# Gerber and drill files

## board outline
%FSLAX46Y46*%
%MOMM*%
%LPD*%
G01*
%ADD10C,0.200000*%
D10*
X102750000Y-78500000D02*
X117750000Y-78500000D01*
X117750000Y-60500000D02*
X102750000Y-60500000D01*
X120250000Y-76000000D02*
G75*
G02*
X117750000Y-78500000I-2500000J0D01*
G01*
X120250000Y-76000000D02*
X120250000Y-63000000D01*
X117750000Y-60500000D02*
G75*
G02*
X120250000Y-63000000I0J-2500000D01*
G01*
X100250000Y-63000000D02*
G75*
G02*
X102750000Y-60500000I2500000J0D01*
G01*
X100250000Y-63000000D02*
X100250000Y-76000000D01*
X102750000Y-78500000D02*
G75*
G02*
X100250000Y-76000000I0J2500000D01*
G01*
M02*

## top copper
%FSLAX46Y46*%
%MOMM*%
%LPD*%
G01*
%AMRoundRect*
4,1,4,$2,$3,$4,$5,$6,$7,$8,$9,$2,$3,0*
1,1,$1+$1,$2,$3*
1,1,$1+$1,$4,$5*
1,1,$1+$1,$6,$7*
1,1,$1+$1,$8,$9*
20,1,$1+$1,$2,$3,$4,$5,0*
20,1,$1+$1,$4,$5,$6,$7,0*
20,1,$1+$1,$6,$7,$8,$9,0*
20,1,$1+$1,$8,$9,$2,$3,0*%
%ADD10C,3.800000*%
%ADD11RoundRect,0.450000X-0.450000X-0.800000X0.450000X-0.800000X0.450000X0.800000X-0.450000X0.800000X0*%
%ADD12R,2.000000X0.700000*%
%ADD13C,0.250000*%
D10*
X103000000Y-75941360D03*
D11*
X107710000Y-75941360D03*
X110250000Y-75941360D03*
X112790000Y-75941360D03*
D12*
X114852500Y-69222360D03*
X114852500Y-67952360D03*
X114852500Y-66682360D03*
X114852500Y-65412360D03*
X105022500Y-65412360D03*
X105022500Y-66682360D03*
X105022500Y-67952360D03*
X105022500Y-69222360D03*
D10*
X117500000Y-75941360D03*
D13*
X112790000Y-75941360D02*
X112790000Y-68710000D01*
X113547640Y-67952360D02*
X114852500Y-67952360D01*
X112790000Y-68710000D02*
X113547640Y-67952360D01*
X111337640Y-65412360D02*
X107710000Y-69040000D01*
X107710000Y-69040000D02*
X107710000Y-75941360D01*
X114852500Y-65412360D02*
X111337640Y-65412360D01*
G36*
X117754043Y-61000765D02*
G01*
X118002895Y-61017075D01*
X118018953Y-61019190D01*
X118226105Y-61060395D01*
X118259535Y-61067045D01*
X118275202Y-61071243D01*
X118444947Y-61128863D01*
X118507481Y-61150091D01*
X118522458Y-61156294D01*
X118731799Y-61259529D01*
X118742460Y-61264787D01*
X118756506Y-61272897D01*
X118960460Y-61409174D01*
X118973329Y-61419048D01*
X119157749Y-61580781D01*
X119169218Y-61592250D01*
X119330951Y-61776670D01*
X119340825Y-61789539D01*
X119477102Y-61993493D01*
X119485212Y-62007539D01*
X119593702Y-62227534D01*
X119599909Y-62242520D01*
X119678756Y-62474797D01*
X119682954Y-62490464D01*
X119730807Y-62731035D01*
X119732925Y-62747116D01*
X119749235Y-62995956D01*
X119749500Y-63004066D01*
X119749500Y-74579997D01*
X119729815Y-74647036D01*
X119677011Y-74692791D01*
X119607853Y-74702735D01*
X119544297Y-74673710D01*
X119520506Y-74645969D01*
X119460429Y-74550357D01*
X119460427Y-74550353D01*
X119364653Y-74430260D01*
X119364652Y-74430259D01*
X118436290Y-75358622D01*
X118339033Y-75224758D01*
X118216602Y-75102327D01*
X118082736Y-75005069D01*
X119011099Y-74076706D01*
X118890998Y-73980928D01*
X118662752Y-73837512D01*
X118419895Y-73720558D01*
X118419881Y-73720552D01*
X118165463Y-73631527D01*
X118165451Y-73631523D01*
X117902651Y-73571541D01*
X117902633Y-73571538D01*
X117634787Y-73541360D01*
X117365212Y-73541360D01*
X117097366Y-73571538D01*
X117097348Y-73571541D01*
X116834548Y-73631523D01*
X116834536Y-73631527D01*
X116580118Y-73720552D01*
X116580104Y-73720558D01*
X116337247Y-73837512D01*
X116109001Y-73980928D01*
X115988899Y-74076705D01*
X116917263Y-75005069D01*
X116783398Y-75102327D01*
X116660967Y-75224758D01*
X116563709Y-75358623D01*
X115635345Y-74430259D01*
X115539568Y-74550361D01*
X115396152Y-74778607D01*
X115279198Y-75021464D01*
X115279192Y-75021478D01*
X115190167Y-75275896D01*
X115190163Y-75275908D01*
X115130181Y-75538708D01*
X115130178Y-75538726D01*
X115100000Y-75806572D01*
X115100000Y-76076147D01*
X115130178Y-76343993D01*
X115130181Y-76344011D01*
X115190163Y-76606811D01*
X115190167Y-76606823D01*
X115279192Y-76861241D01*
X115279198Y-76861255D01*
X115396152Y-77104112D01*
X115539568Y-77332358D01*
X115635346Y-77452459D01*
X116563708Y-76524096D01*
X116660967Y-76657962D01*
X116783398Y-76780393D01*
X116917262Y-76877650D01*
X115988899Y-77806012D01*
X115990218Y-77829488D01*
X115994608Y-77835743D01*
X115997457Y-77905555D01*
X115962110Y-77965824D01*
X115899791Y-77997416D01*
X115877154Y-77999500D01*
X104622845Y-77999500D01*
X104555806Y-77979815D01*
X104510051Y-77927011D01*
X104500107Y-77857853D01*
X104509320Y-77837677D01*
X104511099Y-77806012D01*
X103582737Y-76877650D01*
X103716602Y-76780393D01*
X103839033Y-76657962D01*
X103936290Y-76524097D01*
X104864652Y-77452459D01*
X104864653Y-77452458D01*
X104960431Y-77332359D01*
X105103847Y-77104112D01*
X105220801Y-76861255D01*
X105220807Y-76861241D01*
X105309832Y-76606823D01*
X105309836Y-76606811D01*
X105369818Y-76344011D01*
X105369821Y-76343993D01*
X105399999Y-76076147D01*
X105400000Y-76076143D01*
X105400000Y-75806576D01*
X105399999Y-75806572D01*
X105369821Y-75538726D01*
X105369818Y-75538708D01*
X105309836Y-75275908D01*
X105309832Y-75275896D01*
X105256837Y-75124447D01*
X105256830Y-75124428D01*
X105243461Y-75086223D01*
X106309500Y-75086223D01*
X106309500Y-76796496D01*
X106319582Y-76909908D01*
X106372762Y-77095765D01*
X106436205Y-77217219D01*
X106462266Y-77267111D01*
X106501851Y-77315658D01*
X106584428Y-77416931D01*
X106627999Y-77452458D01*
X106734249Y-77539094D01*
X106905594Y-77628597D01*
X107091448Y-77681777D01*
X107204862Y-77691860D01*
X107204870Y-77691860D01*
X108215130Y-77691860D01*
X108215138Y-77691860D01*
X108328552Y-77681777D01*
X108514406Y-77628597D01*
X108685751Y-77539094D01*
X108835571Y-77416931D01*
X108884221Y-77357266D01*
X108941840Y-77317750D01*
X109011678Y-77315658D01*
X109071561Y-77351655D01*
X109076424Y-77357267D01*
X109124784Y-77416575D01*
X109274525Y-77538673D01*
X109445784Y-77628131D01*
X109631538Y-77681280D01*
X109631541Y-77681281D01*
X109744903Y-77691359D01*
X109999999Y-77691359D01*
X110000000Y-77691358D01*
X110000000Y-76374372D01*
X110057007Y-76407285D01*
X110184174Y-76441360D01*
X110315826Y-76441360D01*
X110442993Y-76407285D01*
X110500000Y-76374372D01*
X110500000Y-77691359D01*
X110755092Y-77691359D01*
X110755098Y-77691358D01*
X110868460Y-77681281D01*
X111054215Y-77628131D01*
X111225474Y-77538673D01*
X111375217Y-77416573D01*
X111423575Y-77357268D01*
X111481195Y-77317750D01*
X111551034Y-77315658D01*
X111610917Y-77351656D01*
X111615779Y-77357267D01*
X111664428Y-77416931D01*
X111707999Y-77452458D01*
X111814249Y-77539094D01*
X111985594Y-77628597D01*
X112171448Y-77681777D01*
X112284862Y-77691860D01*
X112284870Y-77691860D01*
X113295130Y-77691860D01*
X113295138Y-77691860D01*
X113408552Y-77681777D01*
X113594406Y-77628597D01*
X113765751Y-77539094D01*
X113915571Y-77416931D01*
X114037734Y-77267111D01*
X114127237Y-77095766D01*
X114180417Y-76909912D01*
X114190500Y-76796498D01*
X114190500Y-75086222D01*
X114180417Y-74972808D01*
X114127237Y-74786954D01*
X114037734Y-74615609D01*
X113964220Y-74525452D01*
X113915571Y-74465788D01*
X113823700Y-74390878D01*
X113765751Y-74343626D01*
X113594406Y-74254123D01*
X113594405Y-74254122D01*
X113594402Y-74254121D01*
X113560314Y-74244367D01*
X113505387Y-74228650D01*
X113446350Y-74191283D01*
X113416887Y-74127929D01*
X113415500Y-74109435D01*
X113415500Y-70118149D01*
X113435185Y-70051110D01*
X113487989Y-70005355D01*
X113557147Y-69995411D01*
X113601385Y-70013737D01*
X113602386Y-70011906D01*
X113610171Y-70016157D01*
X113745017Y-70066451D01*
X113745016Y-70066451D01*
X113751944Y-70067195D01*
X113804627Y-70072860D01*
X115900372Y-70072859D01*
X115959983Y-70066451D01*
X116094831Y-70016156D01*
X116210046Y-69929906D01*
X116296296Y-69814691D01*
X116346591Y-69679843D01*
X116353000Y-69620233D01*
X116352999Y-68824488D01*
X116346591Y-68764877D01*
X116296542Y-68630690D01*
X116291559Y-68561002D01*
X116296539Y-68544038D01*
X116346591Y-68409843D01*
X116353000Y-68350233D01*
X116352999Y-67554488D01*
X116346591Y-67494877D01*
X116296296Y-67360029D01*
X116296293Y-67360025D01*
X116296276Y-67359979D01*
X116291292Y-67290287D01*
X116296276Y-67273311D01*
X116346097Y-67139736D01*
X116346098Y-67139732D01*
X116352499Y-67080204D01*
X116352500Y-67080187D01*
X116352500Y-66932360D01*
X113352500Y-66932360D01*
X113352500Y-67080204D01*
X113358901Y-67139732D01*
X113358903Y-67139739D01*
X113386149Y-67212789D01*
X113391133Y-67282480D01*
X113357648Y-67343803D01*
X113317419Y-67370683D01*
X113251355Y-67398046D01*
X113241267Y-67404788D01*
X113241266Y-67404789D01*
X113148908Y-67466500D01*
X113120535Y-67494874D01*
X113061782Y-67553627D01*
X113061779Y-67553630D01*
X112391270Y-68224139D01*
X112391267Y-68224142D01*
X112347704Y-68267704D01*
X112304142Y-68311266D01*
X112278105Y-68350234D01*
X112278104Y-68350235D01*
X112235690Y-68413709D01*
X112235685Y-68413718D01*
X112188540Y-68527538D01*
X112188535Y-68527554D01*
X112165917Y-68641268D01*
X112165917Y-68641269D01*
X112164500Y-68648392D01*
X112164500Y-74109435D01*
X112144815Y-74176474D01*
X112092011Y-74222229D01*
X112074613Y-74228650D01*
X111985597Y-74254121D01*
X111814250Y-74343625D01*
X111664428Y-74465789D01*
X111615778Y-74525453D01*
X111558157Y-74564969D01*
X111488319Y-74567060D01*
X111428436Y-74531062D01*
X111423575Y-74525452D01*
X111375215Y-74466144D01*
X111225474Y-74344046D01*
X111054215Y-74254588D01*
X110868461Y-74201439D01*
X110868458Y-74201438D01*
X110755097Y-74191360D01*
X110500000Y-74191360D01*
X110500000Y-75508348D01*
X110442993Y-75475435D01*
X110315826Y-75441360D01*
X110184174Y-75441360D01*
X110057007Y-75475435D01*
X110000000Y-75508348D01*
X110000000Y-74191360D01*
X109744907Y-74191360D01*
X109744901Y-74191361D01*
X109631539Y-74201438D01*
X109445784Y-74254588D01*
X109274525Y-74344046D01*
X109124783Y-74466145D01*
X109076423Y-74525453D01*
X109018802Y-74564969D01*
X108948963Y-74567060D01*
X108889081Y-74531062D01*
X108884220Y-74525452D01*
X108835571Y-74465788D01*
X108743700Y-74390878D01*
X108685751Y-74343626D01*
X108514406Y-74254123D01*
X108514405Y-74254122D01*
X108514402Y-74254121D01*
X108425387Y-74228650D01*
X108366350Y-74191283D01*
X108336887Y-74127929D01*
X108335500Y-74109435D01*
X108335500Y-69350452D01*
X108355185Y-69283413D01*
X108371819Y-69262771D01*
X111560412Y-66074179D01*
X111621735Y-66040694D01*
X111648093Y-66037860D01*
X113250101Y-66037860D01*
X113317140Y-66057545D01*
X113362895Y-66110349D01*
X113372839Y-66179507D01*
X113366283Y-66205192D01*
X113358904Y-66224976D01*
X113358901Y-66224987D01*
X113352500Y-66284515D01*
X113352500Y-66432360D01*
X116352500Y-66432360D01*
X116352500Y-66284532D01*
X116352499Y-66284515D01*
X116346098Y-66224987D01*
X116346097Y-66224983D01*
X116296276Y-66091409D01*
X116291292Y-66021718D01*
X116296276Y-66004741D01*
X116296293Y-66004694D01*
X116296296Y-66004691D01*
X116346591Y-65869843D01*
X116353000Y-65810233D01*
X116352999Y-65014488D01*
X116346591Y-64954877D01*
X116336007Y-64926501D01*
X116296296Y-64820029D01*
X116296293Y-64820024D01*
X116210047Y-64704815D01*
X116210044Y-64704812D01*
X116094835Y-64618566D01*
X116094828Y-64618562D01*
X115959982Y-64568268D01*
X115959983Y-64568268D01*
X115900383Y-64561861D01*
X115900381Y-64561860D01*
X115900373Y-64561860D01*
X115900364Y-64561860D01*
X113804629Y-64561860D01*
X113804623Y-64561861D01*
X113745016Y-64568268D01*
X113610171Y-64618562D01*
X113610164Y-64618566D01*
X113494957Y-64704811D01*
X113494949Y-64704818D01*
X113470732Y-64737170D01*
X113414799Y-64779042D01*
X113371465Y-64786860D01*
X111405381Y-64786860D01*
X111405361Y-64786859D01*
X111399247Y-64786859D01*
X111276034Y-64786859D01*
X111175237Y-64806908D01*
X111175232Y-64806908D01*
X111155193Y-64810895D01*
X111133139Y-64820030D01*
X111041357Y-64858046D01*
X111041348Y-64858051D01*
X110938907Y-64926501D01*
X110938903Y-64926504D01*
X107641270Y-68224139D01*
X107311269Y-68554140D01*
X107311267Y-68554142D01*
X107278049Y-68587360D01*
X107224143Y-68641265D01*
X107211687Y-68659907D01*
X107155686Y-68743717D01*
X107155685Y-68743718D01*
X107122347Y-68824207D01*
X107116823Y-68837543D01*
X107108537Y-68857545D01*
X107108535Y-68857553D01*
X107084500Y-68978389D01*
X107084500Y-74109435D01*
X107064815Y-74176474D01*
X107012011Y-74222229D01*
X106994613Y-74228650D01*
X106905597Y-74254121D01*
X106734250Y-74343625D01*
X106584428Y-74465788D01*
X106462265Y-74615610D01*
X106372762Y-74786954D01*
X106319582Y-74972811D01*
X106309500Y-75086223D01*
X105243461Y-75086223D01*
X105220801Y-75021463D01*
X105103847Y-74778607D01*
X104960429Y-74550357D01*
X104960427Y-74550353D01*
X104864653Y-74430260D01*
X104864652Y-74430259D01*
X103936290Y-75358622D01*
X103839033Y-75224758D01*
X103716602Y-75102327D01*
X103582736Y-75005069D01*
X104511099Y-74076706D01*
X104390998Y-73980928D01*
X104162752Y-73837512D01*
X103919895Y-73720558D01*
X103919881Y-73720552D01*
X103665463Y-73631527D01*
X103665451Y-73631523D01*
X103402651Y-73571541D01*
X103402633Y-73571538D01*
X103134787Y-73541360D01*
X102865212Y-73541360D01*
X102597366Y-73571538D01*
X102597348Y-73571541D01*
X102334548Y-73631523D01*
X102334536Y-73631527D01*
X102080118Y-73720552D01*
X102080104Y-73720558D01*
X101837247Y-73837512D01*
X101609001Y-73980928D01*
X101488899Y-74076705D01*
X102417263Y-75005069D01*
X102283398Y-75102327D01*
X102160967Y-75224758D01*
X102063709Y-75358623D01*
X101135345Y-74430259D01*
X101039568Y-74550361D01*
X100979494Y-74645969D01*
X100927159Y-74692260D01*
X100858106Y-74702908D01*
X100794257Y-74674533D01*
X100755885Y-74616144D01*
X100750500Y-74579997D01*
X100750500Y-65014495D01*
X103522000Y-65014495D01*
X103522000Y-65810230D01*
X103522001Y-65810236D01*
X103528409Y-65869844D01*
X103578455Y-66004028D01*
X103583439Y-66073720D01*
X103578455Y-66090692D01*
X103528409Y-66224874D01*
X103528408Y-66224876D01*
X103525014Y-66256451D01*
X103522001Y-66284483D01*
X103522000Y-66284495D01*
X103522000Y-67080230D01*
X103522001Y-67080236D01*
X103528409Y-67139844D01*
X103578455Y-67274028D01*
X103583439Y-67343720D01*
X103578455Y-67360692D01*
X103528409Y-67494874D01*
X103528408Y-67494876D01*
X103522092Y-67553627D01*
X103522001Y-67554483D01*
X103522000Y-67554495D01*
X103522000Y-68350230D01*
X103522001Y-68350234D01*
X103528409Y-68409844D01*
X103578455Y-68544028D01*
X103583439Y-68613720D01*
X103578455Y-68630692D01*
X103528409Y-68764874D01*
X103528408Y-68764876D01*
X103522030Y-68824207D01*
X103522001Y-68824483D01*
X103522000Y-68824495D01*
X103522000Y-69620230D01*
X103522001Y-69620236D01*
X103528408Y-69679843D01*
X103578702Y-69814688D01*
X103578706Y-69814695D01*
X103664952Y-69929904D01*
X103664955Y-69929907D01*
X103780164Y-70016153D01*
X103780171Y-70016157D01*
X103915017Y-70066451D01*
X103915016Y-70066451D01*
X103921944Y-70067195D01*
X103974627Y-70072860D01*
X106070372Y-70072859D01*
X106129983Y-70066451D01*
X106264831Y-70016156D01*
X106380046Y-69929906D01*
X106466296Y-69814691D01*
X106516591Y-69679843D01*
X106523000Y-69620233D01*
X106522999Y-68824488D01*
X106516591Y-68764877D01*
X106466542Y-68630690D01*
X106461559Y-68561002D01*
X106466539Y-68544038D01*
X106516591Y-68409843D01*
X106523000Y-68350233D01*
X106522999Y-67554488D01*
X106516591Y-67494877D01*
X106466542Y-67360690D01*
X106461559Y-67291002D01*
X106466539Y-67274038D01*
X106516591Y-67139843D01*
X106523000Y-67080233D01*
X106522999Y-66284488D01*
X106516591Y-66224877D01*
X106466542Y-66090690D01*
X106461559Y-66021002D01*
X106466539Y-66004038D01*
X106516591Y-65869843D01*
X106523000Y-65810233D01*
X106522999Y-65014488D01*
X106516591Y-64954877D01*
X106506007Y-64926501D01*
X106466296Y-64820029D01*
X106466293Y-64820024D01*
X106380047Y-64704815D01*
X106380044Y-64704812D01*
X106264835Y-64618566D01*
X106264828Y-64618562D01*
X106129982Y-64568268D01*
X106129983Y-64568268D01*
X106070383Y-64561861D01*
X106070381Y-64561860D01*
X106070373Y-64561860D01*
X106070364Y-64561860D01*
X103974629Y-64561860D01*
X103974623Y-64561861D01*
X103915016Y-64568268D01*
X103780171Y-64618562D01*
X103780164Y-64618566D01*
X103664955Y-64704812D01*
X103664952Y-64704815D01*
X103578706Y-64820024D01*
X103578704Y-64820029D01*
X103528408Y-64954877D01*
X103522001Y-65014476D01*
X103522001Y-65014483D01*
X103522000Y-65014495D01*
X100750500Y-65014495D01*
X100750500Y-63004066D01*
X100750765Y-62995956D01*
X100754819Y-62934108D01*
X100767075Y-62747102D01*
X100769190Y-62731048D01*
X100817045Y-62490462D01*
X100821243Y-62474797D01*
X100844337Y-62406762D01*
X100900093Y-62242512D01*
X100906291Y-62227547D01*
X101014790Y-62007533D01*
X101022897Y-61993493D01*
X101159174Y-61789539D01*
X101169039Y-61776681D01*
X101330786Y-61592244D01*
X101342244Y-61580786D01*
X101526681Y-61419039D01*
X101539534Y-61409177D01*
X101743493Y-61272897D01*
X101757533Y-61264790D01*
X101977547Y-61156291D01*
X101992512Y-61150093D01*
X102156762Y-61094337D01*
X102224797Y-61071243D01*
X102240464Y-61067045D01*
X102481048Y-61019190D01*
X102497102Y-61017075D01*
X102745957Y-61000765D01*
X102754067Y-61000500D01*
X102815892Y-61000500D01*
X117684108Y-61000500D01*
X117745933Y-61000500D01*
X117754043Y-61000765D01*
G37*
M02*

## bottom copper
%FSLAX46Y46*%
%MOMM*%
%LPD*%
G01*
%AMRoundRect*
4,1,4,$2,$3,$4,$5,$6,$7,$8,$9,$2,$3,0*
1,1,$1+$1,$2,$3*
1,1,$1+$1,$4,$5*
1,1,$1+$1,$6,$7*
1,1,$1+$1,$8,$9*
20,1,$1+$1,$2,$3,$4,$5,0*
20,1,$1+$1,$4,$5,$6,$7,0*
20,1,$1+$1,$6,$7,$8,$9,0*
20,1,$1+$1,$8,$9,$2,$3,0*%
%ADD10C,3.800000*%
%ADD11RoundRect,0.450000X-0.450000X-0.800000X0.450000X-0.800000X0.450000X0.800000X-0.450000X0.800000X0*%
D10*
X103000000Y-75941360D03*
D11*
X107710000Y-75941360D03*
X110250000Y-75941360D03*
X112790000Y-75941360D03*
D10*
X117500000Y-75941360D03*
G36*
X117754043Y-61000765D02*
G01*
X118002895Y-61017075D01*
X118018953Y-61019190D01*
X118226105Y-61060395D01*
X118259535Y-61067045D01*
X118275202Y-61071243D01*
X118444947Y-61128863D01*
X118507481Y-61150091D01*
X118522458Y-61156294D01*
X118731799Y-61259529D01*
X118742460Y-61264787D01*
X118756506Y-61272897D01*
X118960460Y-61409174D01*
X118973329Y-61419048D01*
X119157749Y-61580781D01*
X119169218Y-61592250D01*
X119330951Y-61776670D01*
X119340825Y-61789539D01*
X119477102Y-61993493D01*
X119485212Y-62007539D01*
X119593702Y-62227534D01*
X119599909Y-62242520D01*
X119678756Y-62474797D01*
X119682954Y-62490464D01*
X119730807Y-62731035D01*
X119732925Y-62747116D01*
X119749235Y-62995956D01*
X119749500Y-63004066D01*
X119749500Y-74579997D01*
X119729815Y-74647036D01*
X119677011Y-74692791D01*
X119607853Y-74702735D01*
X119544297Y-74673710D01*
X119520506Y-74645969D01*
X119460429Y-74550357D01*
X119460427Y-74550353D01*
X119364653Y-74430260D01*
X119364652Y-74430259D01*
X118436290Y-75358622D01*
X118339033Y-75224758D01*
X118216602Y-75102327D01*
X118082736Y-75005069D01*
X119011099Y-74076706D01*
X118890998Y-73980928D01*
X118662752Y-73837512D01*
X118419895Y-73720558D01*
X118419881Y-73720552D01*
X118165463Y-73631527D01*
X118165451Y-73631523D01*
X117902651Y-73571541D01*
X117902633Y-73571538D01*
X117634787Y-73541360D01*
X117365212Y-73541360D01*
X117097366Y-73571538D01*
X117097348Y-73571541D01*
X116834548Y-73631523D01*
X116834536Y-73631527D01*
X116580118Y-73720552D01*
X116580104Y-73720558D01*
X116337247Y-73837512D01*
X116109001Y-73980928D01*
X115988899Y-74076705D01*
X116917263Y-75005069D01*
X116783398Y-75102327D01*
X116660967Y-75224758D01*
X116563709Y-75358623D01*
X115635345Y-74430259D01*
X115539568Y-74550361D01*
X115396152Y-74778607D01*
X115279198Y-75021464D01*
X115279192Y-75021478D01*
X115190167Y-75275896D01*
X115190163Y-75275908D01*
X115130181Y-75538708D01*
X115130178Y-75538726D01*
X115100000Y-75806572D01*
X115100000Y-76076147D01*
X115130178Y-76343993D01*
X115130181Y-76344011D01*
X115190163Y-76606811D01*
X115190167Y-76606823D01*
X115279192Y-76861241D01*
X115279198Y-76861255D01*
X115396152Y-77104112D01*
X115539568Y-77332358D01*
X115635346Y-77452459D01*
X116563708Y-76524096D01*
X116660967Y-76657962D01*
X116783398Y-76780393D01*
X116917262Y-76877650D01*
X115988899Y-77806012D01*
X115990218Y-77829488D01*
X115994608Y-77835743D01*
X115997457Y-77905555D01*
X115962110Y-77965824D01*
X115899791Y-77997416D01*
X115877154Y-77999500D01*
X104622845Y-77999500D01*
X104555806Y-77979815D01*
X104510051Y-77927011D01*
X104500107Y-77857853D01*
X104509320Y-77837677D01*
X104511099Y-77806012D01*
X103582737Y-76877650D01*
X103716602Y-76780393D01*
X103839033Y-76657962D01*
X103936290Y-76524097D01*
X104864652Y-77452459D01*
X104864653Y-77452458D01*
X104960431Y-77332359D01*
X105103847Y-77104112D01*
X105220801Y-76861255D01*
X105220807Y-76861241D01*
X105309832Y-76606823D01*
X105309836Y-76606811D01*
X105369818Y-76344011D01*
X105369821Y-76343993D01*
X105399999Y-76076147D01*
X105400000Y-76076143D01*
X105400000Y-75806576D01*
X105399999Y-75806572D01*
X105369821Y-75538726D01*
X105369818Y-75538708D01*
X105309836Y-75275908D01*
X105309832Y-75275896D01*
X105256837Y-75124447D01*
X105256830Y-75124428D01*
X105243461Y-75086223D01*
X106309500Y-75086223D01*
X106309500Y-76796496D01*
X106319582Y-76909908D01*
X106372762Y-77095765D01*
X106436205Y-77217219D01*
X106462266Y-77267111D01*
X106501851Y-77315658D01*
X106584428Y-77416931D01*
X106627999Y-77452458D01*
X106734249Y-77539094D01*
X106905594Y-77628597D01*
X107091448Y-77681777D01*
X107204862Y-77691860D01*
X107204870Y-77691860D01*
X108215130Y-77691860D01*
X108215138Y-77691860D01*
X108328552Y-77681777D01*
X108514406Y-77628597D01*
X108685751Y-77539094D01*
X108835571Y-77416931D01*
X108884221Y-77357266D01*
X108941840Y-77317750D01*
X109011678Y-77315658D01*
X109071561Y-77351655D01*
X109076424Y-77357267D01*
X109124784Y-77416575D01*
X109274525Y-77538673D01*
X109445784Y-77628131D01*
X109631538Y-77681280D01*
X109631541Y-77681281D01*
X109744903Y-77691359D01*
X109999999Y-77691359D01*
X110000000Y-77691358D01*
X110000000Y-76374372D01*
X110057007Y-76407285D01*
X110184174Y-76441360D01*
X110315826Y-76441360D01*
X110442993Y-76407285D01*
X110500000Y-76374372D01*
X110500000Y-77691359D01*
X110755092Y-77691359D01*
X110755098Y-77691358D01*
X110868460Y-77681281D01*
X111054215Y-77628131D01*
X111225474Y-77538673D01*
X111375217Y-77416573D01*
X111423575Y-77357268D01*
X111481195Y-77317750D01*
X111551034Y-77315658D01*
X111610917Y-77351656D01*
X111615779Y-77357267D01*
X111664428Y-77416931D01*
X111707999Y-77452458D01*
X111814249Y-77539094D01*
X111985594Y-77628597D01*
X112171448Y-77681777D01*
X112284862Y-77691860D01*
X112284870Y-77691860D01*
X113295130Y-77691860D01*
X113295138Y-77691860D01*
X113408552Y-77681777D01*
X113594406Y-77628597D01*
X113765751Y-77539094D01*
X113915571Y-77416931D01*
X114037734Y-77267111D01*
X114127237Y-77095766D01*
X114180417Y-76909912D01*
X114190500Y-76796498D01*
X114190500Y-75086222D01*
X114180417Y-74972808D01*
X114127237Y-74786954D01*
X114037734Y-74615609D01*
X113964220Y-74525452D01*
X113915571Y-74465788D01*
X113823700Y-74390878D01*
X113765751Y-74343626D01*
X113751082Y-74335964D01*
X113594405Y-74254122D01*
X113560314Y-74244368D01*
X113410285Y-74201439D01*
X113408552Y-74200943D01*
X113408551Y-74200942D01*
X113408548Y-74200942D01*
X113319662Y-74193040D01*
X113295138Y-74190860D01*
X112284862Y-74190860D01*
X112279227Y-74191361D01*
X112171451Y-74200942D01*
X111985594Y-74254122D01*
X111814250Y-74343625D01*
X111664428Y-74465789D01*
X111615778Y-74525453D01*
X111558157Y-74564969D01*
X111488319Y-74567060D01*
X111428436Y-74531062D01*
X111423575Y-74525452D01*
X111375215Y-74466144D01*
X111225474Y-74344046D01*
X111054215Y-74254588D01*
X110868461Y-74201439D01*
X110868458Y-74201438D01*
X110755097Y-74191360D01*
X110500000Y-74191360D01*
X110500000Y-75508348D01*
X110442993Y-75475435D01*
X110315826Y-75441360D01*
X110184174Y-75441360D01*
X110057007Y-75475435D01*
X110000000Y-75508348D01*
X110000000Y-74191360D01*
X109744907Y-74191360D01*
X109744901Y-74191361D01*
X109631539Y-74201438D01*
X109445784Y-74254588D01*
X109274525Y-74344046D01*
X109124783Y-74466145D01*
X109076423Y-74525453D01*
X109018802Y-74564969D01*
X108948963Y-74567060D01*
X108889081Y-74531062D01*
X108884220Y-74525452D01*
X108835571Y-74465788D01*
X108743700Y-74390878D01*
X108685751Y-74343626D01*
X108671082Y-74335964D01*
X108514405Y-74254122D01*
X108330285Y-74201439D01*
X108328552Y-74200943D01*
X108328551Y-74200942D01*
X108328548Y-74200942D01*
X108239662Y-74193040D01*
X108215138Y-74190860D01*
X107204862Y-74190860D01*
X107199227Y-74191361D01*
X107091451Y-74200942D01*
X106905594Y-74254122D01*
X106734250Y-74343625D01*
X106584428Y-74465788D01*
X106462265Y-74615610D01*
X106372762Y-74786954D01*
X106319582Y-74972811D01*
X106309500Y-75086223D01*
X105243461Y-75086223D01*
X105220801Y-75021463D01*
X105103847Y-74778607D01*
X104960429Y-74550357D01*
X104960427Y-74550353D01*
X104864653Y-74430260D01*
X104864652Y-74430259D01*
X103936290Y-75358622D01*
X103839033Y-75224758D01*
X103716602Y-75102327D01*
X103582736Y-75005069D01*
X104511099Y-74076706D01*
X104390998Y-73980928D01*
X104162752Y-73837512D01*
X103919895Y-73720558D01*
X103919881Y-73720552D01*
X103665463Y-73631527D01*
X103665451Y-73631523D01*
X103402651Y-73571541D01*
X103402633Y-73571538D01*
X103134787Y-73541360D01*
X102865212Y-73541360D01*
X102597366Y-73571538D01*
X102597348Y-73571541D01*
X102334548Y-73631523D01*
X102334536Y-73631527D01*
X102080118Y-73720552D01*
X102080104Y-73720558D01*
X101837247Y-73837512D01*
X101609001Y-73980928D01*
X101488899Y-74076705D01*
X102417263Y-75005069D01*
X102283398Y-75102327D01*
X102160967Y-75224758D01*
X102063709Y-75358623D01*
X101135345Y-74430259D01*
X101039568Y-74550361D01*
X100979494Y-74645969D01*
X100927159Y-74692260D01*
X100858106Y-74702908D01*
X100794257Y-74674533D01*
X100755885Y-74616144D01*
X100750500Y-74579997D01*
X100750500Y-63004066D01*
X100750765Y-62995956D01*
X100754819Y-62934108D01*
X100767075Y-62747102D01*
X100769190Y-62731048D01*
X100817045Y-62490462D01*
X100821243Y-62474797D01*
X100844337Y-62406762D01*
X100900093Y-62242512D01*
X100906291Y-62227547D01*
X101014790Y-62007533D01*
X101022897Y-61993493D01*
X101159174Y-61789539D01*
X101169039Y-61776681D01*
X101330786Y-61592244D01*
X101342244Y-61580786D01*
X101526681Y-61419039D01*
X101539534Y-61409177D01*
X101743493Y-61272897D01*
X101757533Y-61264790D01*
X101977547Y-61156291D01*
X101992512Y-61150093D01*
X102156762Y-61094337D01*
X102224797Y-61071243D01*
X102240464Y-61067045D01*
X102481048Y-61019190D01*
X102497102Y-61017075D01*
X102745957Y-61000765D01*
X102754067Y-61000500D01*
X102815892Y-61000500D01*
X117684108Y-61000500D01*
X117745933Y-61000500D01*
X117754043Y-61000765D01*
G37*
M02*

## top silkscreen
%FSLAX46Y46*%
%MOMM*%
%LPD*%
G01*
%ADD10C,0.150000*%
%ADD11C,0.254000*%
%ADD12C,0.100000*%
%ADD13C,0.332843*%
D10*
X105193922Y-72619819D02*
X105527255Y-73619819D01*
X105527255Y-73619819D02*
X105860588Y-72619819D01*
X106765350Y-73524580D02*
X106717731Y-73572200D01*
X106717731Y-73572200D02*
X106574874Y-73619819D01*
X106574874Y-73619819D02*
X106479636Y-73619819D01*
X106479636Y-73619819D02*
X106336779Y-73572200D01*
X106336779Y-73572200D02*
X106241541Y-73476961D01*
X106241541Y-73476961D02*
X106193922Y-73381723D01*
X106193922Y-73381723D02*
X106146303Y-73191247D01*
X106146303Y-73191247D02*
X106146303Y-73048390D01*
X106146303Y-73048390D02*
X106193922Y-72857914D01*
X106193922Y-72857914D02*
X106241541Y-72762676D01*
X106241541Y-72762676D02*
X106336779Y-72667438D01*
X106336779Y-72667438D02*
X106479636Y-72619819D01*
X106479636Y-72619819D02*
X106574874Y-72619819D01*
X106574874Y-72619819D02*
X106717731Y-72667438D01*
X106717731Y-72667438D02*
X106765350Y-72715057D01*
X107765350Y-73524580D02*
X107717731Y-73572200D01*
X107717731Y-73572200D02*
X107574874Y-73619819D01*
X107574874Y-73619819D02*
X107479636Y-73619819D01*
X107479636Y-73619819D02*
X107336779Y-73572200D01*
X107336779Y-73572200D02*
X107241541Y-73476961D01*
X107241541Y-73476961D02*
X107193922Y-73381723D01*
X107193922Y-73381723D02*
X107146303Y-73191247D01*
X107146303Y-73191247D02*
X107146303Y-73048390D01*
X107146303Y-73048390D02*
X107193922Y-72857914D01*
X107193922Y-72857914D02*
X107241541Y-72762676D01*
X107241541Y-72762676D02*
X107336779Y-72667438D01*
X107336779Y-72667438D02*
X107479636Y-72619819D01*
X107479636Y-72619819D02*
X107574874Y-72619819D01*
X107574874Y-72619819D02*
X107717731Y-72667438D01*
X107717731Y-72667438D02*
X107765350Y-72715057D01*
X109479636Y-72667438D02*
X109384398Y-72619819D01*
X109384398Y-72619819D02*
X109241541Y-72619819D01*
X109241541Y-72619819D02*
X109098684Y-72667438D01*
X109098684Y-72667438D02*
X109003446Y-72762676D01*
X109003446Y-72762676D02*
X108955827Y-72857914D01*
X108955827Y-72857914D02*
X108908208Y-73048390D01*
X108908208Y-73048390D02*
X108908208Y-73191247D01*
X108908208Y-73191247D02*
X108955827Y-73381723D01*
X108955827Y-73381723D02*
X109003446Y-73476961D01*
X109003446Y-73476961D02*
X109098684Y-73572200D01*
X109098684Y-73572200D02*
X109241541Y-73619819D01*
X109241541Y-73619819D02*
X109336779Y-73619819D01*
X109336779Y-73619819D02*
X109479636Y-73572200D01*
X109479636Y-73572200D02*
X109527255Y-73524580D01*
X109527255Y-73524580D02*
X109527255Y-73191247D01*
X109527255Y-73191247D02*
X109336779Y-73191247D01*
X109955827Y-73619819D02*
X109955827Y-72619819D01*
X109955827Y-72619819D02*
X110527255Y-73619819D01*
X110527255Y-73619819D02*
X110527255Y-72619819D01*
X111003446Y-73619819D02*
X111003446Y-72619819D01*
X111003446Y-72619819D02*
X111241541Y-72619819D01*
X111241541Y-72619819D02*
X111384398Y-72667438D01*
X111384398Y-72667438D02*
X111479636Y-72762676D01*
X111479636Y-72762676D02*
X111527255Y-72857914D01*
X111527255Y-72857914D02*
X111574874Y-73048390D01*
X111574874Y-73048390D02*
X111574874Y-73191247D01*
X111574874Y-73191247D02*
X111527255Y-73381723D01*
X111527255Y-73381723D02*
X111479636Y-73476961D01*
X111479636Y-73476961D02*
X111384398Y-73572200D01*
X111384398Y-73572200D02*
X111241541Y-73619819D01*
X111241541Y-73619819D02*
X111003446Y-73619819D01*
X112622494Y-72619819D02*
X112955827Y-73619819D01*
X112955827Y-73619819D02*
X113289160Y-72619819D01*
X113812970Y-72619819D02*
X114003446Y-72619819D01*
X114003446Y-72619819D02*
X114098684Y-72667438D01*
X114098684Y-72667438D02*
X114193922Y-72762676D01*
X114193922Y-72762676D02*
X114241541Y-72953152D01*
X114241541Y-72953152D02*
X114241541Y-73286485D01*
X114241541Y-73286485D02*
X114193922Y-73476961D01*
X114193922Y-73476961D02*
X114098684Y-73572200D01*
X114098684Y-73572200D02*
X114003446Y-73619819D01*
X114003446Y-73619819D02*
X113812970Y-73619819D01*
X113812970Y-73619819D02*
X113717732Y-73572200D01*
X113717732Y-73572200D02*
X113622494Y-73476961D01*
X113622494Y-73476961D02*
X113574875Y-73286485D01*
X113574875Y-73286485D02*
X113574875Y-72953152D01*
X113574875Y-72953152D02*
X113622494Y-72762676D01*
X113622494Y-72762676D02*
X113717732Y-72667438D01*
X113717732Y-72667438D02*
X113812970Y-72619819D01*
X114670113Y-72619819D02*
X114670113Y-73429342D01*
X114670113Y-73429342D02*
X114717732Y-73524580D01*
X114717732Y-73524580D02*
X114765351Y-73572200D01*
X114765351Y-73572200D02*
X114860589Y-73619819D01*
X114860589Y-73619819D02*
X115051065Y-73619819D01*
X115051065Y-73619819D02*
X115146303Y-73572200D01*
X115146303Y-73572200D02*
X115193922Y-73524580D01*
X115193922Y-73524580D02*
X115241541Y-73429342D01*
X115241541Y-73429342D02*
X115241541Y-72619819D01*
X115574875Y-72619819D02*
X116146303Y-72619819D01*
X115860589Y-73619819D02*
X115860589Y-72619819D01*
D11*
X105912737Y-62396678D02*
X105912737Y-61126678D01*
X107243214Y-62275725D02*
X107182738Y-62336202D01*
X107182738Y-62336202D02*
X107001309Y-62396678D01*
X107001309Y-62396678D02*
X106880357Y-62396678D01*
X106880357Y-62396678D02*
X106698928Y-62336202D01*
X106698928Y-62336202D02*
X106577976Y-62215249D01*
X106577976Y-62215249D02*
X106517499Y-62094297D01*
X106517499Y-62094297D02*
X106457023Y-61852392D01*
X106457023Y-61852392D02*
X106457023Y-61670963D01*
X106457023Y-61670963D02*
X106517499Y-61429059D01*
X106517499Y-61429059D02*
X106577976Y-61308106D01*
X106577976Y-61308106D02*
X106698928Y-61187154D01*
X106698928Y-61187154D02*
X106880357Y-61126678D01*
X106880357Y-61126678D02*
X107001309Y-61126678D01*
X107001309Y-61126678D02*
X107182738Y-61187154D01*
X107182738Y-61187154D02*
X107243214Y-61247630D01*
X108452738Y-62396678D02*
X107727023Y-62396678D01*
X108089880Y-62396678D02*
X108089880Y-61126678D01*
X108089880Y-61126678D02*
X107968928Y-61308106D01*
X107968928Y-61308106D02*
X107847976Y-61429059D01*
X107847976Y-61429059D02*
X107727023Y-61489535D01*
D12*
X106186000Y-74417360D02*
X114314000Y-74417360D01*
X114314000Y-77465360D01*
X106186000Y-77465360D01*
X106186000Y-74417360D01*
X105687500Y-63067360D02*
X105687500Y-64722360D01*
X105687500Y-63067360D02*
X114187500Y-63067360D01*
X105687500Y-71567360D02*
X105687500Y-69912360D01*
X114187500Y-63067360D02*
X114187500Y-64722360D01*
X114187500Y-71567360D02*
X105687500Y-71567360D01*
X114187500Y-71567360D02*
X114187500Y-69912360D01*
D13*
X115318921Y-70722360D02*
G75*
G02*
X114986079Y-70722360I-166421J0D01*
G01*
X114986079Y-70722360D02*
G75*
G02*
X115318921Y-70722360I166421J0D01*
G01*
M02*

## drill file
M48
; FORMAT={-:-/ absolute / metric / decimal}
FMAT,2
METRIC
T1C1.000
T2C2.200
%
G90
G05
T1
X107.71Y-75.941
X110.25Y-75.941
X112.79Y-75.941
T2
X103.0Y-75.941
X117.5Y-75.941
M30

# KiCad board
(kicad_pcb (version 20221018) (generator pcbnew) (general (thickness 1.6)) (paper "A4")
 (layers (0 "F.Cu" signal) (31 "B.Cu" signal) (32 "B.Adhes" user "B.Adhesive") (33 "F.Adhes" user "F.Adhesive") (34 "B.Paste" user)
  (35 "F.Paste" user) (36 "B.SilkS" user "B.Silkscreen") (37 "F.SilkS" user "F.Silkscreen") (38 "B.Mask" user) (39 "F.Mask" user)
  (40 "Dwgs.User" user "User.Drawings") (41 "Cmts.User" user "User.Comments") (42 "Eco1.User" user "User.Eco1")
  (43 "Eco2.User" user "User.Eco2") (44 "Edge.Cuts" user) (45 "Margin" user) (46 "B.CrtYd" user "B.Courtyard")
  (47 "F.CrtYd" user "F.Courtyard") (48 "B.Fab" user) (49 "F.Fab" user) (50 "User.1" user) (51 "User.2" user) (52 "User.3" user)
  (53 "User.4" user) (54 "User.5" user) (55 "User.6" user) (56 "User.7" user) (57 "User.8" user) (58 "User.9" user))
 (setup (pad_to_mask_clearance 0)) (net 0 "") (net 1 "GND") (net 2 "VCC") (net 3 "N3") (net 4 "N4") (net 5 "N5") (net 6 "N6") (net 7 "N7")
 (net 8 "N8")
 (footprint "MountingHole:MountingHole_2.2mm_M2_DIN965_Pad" (layer "F.Cu") (at 103 75.94136)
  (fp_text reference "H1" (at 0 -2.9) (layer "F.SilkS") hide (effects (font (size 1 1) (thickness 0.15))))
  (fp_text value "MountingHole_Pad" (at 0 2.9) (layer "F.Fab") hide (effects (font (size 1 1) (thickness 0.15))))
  (pad "1" thru_hole circle (at 0 0) (size 3.8 3.8) (drill 2.2) (layers "*.Cu" "*.Mask") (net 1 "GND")))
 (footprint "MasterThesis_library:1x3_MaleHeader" (layer "F.Cu") (at 110.25 75.94136)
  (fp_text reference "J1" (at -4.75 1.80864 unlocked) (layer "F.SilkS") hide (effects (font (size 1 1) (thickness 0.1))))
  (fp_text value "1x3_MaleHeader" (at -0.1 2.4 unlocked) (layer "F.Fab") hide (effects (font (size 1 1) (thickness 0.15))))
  (fp_rect (start -4.064 -1.524) (end 4.064 1.524) (stroke (width 0.1) (type default)) (fill none) (layer "F.SilkS"))
  (pad "1" thru_hole roundrect (at -2.54 0) (size 1.8 2.5) (drill 1) (layers "*.Cu" "*.Mask") (roundrect_rratio 0.25) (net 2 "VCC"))
  (pad "2" thru_hole roundrect (at 0 0) (size 1.8 2.5) (drill 1) (layers "*.Cu" "*.Mask") (roundrect_rratio 0.25) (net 1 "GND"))
  (pad "3" thru_hole roundrect (at 2.54 0) (size 1.8 2.5) (drill 1) (layers "*.Cu" "*.Mask") (roundrect_rratio 0.25) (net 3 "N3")))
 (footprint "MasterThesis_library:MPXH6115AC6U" (layer "F.Cu") (at 114.8525 69.22236)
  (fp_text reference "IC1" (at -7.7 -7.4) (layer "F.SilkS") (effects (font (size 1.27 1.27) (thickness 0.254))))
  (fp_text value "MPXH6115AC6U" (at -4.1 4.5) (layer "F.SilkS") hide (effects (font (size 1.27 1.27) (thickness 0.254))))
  (fp_line (start -9.165 -6.155) (end -9.165 -4.5) (stroke (width 0.1) (type solid)) (layer "F.SilkS"))
  (fp_line (start -9.165 -6.155) (end -0.665 -6.155) (stroke (width 0.1) (type solid)) (layer "F.SilkS"))
  (fp_line (start -9.165 2.345) (end -9.165 0.69) (stroke (width 0.1) (type solid)) (layer "F.SilkS"))
  (fp_line (start -0.665 -6.155) (end -0.665 -4.5) (stroke (width 0.1) (type solid)) (layer "F.SilkS"))
  (fp_line (start -0.665 2.345) (end -9.165 2.345) (stroke (width 0.1) (type solid)) (layer "F.SilkS"))
  (fp_line (start -0.665 2.345) (end -0.665 0.69) (stroke (width 0.1) (type solid)) (layer "F.SilkS"))
  (fp_circle (center 0.3 1.5) (end 0.582843 1.5) (stroke (width 0.1) (type solid)) (fill solid) (layer "F.SilkS"))
  (pad "1" smd rect (at 0 0 90) (size 0.7 2) (layers "F.Cu" "F.Paste" "F.Mask") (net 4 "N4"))
  (pad "2" smd rect (at 0 -1.27 90) (size 0.7 2) (layers "F.Cu" "F.Paste" "F.Mask") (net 3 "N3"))
  (pad "3" smd rect (at 0 -2.54 90) (size 0.7 2) (layers "F.Cu" "F.Paste" "F.Mask") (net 1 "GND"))
  (pad "4" smd rect (at 0 -3.81 90) (size 0.7 2) (layers "F.Cu" "F.Paste" "F.Mask") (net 2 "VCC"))
  (pad "5" smd rect (at -9.83 -3.81 90) (size 0.7 2) (layers "F.Cu" "F.Paste" "F.Mask") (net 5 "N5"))
  (pad "6" smd rect (at -9.83 -2.54 90) (size 0.7 2) (layers "F.Cu" "F.Paste" "F.Mask") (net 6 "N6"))
  (pad "7" smd rect (at -9.83 -1.27 90) (size 0.7 2) (layers "F.Cu" "F.Paste" "F.Mask") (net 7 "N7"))
  (pad "8" smd rect (at -9.83 0 90) (size 0.7 2) (layers "F.Cu" "F.Paste" "F.Mask") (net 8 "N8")))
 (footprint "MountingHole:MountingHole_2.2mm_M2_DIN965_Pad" (layer "F.Cu") (at 117.5 75.94136)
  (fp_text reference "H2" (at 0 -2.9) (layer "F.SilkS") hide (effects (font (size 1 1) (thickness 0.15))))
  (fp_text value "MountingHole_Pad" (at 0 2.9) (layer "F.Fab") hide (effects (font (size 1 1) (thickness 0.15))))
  (pad "1" thru_hole circle (at 0 0) (size 3.8 3.8) (drill 2.2) (layers "*.Cu" "*.Mask") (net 1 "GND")))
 (gr_line locked (start 102.75 78.5) (end 117.75 78.5) (stroke (width 0.2) (type solid)) (layer "Edge.Cuts"))
 (gr_line locked (start 117.75 60.5) (end 102.75 60.5) (stroke (width 0.2) (type solid)) (layer "Edge.Cuts"))
 (gr_arc locked (start 120.25 76) (mid 119.517767 77.767767) (end 117.75 78.5) (stroke (width 0.2) (type solid)) (layer "Edge.Cuts"))
 (gr_line locked (start 120.25 76) (end 120.25 63) (stroke (width 0.2) (type solid)) (layer "Edge.Cuts"))
 (gr_arc locked (start 117.75 60.5) (mid 119.517767 61.232233) (end 120.25 63) (stroke (width 0.2) (type solid)) (layer "Edge.Cuts"))
 (gr_arc locked (start 100.25 63) (mid 100.982233 61.232233) (end 102.75 60.5) (stroke (width 0.2) (type solid)) (layer "Edge.Cuts"))
 (gr_line locked (start 100.25 63) (end 100.25 76) (stroke (width 0.2) (type solid)) (layer "Edge.Cuts"))
 (gr_arc locked (start 102.75 78.5) (mid 100.982233 77.767767) (end 100.25 76) (stroke (width 0.2) (type solid)) (layer "Edge.Cuts"))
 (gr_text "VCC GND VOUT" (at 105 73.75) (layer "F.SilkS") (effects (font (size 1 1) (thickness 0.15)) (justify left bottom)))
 (segment (start 112.79 75.94136) (end 112.79 68.71) (width 0.25) (layer "F.Cu") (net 3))
 (segment (start 113.54764 67.95236) (end 114.8525 67.95236) (width 0.25) (layer "F.Cu") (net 3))
 (segment (start 112.79 68.71) (end 113.54764 67.95236) (width 0.25) (layer "F.Cu") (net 3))
 (segment (start 111.33764 65.41236) (end 107.71 69.04) (width 0.25) (layer "F.Cu") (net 2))
 (segment (start 107.71 69.04) (end 107.71 75.94136) (width 0.25) (layer "F.Cu") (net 2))
 (segment (start 114.8525 65.41236) (end 111.33764 65.41236) (width 0.25) (layer "F.Cu") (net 2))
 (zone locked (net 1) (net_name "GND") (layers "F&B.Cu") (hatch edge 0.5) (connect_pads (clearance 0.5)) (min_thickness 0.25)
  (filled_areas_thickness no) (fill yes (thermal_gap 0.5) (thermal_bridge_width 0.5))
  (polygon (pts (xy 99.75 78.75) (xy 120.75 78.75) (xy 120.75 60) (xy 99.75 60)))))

